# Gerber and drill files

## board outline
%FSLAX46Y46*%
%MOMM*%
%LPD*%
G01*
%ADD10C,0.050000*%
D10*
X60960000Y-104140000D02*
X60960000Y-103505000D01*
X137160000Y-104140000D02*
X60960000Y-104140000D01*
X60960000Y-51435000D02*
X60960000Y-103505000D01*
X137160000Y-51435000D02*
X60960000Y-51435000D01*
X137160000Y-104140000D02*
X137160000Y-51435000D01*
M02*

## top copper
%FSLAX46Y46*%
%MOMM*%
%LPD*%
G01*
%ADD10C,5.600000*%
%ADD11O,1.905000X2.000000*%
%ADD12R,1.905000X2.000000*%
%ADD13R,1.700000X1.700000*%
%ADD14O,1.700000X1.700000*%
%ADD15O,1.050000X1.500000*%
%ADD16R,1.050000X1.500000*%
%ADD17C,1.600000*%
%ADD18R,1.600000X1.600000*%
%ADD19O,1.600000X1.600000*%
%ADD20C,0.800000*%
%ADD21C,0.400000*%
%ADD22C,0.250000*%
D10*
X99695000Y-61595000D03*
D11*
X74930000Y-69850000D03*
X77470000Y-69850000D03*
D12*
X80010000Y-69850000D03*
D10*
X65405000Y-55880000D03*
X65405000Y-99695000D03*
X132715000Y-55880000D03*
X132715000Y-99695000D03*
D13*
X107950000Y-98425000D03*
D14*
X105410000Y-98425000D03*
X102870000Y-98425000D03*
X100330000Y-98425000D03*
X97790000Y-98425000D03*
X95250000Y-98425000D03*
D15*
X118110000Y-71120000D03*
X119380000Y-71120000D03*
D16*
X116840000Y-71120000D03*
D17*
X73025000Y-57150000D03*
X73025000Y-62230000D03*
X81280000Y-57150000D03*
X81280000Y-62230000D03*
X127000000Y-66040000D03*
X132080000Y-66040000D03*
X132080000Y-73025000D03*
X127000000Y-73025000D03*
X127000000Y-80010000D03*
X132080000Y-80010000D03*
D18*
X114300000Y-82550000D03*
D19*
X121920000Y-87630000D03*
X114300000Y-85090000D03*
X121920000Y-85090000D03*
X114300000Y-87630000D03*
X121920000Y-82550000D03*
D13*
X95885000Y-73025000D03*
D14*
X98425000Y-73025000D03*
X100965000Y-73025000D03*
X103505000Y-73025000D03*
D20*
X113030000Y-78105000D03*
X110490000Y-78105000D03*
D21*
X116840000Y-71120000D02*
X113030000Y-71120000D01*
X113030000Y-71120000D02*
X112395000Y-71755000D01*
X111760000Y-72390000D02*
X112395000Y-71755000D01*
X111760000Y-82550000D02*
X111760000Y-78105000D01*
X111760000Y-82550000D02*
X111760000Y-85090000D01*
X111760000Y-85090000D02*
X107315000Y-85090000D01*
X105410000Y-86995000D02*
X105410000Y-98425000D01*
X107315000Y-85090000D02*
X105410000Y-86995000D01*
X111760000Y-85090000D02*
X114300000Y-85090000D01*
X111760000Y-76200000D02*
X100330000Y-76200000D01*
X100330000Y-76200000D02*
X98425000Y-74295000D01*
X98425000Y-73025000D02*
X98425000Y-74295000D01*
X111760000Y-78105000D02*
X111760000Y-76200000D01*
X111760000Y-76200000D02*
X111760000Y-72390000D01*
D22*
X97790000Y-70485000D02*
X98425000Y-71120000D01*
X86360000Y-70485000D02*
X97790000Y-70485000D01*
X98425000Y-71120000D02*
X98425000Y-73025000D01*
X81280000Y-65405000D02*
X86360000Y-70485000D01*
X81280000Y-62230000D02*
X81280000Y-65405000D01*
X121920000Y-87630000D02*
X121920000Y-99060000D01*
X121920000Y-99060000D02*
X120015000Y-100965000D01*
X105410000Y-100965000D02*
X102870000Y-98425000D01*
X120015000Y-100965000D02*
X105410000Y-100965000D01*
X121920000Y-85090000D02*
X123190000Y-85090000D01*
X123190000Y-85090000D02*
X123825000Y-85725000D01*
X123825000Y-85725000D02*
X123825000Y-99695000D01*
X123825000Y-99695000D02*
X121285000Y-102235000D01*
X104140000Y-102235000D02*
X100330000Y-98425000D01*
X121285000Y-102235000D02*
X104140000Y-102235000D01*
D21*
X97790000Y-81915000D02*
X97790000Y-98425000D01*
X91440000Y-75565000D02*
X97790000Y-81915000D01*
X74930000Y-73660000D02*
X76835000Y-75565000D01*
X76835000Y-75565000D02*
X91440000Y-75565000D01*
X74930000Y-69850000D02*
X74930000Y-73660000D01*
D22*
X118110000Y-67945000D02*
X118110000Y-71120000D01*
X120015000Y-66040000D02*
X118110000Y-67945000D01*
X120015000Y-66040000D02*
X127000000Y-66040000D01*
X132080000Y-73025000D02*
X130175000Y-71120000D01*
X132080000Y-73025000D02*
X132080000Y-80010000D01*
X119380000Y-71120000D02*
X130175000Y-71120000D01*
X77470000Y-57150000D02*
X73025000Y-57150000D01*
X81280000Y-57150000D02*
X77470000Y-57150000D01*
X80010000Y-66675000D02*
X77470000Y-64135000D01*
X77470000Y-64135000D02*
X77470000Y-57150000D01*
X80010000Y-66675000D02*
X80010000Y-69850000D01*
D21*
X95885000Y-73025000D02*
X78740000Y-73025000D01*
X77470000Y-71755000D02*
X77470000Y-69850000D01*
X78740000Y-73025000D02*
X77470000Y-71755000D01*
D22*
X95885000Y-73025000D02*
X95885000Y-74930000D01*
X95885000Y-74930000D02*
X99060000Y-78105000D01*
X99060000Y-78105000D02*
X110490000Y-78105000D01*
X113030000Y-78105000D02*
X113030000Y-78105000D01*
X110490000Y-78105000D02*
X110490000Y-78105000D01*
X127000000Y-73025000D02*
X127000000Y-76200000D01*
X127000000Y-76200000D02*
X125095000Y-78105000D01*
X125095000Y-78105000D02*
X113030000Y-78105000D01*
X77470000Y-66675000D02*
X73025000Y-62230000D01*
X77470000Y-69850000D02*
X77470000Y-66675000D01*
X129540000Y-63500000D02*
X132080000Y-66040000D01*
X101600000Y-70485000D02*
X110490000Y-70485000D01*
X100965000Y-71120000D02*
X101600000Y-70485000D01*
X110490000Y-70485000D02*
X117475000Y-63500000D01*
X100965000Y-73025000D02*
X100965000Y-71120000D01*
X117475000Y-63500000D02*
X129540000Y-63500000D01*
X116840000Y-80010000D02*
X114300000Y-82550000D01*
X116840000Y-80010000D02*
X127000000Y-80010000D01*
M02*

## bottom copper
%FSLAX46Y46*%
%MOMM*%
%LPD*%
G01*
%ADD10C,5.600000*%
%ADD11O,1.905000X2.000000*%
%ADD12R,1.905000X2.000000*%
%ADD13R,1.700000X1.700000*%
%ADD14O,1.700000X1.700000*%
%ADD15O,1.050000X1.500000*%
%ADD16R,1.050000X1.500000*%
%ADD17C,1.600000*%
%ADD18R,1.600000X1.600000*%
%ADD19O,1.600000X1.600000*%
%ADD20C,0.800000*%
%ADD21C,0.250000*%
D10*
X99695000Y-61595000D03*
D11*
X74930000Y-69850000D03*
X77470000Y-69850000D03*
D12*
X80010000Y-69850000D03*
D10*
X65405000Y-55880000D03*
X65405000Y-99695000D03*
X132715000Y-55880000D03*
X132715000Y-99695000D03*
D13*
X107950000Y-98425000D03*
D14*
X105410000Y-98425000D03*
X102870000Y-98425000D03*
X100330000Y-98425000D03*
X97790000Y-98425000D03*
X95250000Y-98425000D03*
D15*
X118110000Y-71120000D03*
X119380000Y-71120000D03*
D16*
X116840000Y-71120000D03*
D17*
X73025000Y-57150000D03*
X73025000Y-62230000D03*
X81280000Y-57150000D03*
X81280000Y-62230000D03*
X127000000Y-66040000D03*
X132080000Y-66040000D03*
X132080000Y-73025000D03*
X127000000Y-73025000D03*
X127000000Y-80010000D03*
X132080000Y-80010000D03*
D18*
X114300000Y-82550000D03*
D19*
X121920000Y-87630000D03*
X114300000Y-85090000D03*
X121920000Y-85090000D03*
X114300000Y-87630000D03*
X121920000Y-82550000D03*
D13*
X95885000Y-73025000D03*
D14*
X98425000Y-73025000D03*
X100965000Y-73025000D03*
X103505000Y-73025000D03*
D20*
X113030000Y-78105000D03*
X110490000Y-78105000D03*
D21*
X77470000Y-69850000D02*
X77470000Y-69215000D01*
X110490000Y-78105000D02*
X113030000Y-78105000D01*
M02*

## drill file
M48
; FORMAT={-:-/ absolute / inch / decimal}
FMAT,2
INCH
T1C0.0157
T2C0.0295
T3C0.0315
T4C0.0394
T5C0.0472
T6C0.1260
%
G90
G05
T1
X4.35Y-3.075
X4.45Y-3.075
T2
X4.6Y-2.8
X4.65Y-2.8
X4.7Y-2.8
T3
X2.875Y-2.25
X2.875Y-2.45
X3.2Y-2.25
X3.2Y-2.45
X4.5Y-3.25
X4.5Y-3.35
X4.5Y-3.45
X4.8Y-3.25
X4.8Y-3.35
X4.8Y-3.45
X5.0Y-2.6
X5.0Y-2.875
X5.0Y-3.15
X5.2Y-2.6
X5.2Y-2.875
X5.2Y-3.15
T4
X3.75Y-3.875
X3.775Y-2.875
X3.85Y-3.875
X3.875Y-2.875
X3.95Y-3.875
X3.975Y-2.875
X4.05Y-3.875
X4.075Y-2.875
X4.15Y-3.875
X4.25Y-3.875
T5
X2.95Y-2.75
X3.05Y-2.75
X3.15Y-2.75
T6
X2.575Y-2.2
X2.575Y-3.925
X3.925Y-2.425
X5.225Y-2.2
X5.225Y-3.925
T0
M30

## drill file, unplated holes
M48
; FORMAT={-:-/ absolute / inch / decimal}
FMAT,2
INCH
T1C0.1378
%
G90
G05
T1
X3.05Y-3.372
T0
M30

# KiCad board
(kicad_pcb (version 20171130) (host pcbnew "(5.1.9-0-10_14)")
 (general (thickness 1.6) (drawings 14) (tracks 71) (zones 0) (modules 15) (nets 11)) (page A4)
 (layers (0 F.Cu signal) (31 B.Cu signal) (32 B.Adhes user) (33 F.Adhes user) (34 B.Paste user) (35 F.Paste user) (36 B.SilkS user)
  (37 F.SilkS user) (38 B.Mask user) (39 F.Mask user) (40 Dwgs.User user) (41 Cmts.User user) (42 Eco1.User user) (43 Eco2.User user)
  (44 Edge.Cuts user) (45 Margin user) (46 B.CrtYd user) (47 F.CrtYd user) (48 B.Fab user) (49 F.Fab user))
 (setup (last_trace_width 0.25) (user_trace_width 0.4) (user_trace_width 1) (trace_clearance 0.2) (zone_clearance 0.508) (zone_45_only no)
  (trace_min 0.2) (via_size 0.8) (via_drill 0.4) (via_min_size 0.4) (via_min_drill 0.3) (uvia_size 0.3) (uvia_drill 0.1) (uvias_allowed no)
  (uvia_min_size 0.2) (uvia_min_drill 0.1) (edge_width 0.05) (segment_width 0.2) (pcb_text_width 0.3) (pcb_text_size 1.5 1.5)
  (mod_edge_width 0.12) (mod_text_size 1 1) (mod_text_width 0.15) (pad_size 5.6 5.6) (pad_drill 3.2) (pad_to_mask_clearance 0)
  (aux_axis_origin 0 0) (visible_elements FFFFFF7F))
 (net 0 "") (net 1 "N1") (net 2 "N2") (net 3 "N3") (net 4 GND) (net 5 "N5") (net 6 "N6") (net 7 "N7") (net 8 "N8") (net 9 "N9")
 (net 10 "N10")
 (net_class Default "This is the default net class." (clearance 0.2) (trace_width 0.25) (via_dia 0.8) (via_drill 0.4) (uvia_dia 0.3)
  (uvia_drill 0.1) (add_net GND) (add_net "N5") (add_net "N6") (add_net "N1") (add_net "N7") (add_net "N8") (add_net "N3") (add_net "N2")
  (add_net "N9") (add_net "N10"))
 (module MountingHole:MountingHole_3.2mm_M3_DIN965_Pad (layer F.Cu) (at 99.695 61.595)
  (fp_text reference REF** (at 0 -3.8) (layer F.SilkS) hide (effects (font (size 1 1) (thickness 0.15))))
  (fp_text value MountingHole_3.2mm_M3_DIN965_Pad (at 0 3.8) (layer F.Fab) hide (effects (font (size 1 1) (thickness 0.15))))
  (pad "" thru_hole circle (at 0 0) (size 5.6 5.6) (drill 3.2) (layers *.Cu *.Mask)))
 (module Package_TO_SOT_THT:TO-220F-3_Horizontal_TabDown (layer F.Cu) (at 80.01 69.85 180)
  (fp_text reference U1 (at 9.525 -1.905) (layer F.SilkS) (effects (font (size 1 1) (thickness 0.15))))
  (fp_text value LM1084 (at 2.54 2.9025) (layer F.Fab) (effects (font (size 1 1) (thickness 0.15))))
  (pad 3 thru_hole oval (at 5.08 0 180) (size 1.905 2) (drill 1.2) (layers *.Cu *.Mask) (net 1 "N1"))
  (pad 2 thru_hole oval (at 2.54 0 180) (size 1.905 2) (drill 1.2) (layers *.Cu *.Mask) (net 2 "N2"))
  (pad 1 thru_hole rect (at 0 0 180) (size 1.905 2) (drill 1.2) (layers *.Cu *.Mask) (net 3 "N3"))
  (pad "" np_thru_hole oval (at 2.54 -15.8 180) (size 3.5 3.5) (drill 3.5) (layers *.Cu *.Mask)))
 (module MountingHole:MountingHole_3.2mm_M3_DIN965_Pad (layer F.Cu) (at 65.405 55.88)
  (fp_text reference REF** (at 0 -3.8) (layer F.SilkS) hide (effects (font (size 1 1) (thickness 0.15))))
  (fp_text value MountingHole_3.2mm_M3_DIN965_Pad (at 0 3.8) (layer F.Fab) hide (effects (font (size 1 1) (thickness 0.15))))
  (pad "" thru_hole circle (at 0 0) (size 5.6 5.6) (drill 3.2) (layers *.Cu *.Mask)))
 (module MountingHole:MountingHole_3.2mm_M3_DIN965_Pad (layer F.Cu) (at 65.405 99.695)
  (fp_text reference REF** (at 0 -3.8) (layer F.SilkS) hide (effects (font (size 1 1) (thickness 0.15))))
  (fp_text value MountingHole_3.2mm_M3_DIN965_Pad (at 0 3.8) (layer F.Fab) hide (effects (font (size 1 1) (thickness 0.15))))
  (pad "" thru_hole circle (at 0 0) (size 5.6 5.6) (drill 3.2) (layers *.Cu *.Mask)))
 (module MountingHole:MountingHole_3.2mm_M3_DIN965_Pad (layer F.Cu) (at 132.715 55.88)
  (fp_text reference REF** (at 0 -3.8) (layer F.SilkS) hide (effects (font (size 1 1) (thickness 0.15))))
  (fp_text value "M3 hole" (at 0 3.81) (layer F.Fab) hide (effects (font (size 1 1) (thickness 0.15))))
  (pad "" thru_hole circle (at 0 0) (size 5.6 5.6) (drill 3.2) (layers *.Cu *.Mask)))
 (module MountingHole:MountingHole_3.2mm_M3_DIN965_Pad (layer F.Cu) (at 132.715 99.695)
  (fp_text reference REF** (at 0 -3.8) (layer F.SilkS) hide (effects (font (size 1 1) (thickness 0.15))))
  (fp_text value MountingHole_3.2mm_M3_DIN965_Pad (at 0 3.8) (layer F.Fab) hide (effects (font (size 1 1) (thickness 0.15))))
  (pad "" thru_hole circle (at 0 0) (size 5.6 5.6) (drill 3.2) (layers *.Cu *.Mask)))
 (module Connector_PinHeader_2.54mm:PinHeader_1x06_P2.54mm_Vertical (layer F.Cu) (at 107.95 98.425 270)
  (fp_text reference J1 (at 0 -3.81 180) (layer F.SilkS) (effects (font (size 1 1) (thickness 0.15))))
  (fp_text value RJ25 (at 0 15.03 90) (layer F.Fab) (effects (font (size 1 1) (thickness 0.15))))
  (pad 1 thru_hole rect (at 0 0 270) (size 1.7 1.7) (drill 1) (layers *.Cu *.Mask))
  (pad 2 thru_hole oval (at 0 2.54 270) (size 1.7 1.7) (drill 1) (layers *.Cu *.Mask) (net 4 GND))
  (pad 3 thru_hole oval (at 0 5.08 270) (size 1.7 1.7) (drill 1) (layers *.Cu *.Mask) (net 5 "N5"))
  (pad 4 thru_hole oval (at 0 7.62 270) (size 1.7 1.7) (drill 1) (layers *.Cu *.Mask) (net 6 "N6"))
  (pad 5 thru_hole oval (at 0 10.16 270) (size 1.7 1.7) (drill 1) (layers *.Cu *.Mask) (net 1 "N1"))
  (pad 6 thru_hole oval (at 0 12.7 270) (size 1.7 1.7) (drill 1) (layers *.Cu *.Mask)))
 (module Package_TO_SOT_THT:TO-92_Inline (layer F.Cu) (at 116.84 71.12)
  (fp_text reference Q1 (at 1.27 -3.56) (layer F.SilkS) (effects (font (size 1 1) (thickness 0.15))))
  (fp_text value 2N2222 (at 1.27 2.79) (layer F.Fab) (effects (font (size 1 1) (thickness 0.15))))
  (pad 2 thru_hole oval (at 1.27 0) (size 1.05 1.5) (drill 0.75) (layers *.Cu *.Mask) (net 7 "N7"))
  (pad 3 thru_hole oval (at 2.54 0) (size 1.05 1.5) (drill 0.75) (layers *.Cu *.Mask) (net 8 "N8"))
  (pad 1 thru_hole rect (at 0 0) (size 1.05 1.5) (drill 0.75) (layers *.Cu *.Mask) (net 4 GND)))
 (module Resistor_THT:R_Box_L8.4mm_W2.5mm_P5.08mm (layer F.Cu) (at 73.025 57.15 270)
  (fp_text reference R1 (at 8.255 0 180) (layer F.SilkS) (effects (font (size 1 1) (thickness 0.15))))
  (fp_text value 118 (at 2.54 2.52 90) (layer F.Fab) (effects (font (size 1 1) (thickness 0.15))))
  (pad 1 thru_hole circle (at 0 0 270) (size 1.6 1.6) (drill 0.8) (layers *.Cu *.Mask) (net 3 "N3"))
  (pad 2 thru_hole circle (at 5.08 0 270) (size 1.6 1.6) (drill 0.8) (layers *.Cu *.Mask) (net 2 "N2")))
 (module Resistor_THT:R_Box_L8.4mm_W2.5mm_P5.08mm (layer F.Cu) (at 81.28 62.23 90)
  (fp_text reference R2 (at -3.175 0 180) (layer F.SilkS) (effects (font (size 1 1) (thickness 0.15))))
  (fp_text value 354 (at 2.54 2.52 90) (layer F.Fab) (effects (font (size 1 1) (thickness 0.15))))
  (pad 2 thru_hole circle (at 5.08 0 90) (size 1.6 1.6) (drill 0.8) (layers *.Cu *.Mask) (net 3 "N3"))
  (pad 1 thru_hole circle (at 0 0 90) (size 1.6 1.6) (drill 0.8) (layers *.Cu *.Mask) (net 4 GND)))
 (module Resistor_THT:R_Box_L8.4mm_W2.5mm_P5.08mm (layer F.Cu) (at 127 66.04)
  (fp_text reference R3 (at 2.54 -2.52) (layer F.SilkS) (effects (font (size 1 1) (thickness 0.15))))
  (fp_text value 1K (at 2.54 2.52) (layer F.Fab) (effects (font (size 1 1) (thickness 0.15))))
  (pad 1 thru_hole circle (at 0 0) (size 1.6 1.6) (drill 0.8) (layers *.Cu *.Mask) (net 7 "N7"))
  (pad 2 thru_hole circle (at 5.08 0) (size 1.6 1.6) (drill 0.8) (layers *.Cu *.Mask) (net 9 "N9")))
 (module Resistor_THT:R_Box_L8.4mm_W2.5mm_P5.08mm (layer F.Cu) (at 127 73.025)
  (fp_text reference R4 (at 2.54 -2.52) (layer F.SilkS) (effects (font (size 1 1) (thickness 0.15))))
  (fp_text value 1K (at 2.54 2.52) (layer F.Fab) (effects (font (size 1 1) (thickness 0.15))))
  (pad 2 thru_hole circle (at 5.08 0) (size 1.6 1.6) (drill 0.8) (layers *.Cu *.Mask) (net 8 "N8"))
  (pad 1 thru_hole circle (at 0 0) (size 1.6 1.6) (drill 0.8) (layers *.Cu *.Mask) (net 2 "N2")))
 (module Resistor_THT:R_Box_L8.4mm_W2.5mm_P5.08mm (layer F.Cu) (at 127 80.01)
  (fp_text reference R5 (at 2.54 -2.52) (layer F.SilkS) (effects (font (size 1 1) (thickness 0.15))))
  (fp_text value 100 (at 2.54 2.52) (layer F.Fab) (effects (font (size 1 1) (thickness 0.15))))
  (pad 1 thru_hole circle (at 0 0) (size 1.6 1.6) (drill 0.8) (layers *.Cu *.Mask) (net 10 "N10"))
  (pad 2 thru_hole circle (at 5.08 0) (size 1.6 1.6) (drill 0.8) (layers *.Cu *.Mask) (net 8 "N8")))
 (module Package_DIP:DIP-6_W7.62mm (layer F.Cu) (at 114.3 82.55)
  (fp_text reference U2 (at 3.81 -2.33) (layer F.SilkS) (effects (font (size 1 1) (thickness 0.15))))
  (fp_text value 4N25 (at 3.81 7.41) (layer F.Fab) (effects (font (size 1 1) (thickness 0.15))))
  (pad 1 thru_hole rect (at 0 0) (size 1.6 1.6) (drill 0.8) (layers *.Cu *.Mask) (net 10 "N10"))
  (pad 4 thru_hole oval (at 7.62 5.08) (size 1.6 1.6) (drill 0.8) (layers *.Cu *.Mask) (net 5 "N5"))
  (pad 2 thru_hole oval (at 0 2.54) (size 1.6 1.6) (drill 0.8) (layers *.Cu *.Mask) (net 4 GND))
  (pad 5 thru_hole oval (at 7.62 2.54) (size 1.6 1.6) (drill 0.8) (layers *.Cu *.Mask) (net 6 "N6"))
  (pad 3 thru_hole oval (at 0 5.08) (size 1.6 1.6) (drill 0.8) (layers *.Cu *.Mask))
  (pad 6 thru_hole oval (at 7.62 0) (size 1.6 1.6) (drill 0.8) (layers *.Cu *.Mask)))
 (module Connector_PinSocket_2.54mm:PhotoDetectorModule (layer F.Cu) (at 95.885 73.025 90)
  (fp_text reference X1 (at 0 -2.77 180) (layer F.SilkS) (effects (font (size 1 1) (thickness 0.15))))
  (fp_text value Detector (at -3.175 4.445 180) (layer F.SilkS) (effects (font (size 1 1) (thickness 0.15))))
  (pad 1 thru_hole rect (at 0 0 90) (size 1.7 1.7) (drill 1) (layers *.Cu *.Mask) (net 2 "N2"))
  (pad 2 thru_hole oval (at 0 2.54 90) (size 1.7 1.7) (drill 1) (layers *.Cu *.Mask) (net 4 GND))
  (pad 3 thru_hole oval (at 0 5.08 90) (size 1.7 1.7) (drill 1) (layers *.Cu *.Mask) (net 9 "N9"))
  (pad 4 thru_hole oval (at 0 7.62 90) (size 1.7 1.7) (drill 1) (layers *.Cu *.Mask)))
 (gr_line (start 60.96 104.14) (end 60.96 103.505) (layer Edge.Cuts) (width 0.05))
 (gr_line (start 137.16 104.14) (end 60.96 104.14) (layer Edge.Cuts) (width 0.05))
 (gr_line (start 60.96 51.435) (end 60.96 103.505) (layer Edge.Cuts) (width 0.05))
 (gr_line (start 137.16 51.435) (end 60.96 51.435) (layer Edge.Cuts) (width 0.05))
 (gr_line (start 137.16 104.14) (end 137.16 51.435) (layer Edge.Cuts) (width 0.05))
 (segment (start 116.84 71.12) (end 113.03 71.12) (width 0.4) (layer F.Cu) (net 4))
 (segment (start 113.03 71.12) (end 112.395 71.755) (width 0.4) (layer F.Cu) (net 4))
 (segment (start 111.76 72.39) (end 112.395 71.755) (width 0.4) (layer F.Cu) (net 4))
 (segment (start 111.76 82.55) (end 111.76 78.105) (width 0.4) (layer F.Cu) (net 4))
 (segment (start 111.76 82.55) (end 111.76 85.09) (width 0.4) (layer F.Cu) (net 4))
 (segment (start 111.76 85.09) (end 107.315 85.09) (width 0.4) (layer F.Cu) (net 4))
 (segment (start 105.41 86.995) (end 105.41 98.425) (width 0.4) (layer F.Cu) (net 4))
 (segment (start 107.315 85.09) (end 105.41 86.995) (width 0.4) (layer F.Cu) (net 4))
 (segment (start 111.76 85.09) (end 114.3 85.09) (width 0.4) (layer F.Cu) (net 4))
 (segment (start 111.76 76.2) (end 100.33 76.2) (width 0.4) (layer F.Cu) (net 4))
 (segment (start 100.33 76.2) (end 98.425 74.295) (width 0.4) (layer F.Cu) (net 4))
 (segment (start 98.425 73.025) (end 98.425 74.295) (width 0.4) (layer F.Cu) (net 4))
 (segment (start 111.76 78.105) (end 111.76 76.2) (width 0.4) (layer F.Cu) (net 4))
 (segment (start 111.76 76.2) (end 111.76 72.39) (width 0.4) (layer F.Cu) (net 4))
 (segment (start 97.79 70.485) (end 98.425 71.12) (width 0.25) (layer F.Cu) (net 4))
 (segment (start 86.36 70.485) (end 97.79 70.485) (width 0.25) (layer F.Cu) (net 4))
 (segment (start 98.425 71.12) (end 98.425 73.025) (width 0.25) (layer F.Cu) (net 4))
 (segment (start 81.28 65.405) (end 86.36 70.485) (width 0.25) (layer F.Cu) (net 4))
 (segment (start 81.28 62.23) (end 81.28 65.405) (width 0.25) (layer F.Cu) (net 4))
 (segment (start 121.92 87.63) (end 121.92 99.06) (width 0.25) (layer F.Cu) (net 5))
 (segment (start 121.92 99.06) (end 120.015 100.965) (width 0.25) (layer F.Cu) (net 5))
 (segment (start 105.41 100.965) (end 102.87 98.425) (width 0.25) (layer F.Cu) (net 5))
 (segment (start 120.015 100.965) (end 105.41 100.965) (width 0.25) (layer F.Cu) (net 5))
 (segment (start 121.92 85.09) (end 123.19 85.09) (width 0.25) (layer F.Cu) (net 6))
 (segment (start 123.19 85.09) (end 123.825 85.725) (width 0.25) (layer F.Cu) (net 6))
 (segment (start 123.825 85.725) (end 123.825 99.695) (width 0.25) (layer F.Cu) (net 6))
 (segment (start 123.825 99.695) (end 121.285 102.235) (width 0.25) (layer F.Cu) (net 6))
 (segment (start 104.14 102.235) (end 100.33 98.425) (width 0.25) (layer F.Cu) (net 6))
 (segment (start 121.285 102.235) (end 104.14 102.235) (width 0.25) (layer F.Cu) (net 6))
 (segment (start 97.79 81.915) (end 97.79 98.425) (width 0.4) (layer F.Cu) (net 1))
 (segment (start 91.44 75.565) (end 97.79 81.915) (width 0.4) (layer F.Cu) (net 1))
 (segment (start 74.93 73.66) (end 76.835 75.565) (width 0.4) (layer F.Cu) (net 1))
 (segment (start 76.835 75.565) (end 91.44 75.565) (width 0.4) (layer F.Cu) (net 1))
 (segment (start 74.93 69.85) (end 74.93 73.66) (width 0.4) (layer F.Cu) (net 1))
 (segment (start 118.11 67.945) (end 118.11 71.12) (width 0.25) (layer F.Cu) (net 7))
 (segment (start 120.015 66.04) (end 118.11 67.945) (width 0.25) (layer F.Cu) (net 7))
 (segment (start 120.015 66.04) (end 127 66.04) (width 0.25) (layer F.Cu) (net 7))
 (segment (start 132.08 73.025) (end 130.175 71.12) (width 0.25) (layer F.Cu) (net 8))
 (segment (start 132.08 73.025) (end 132.08 80.01) (width 0.25) (layer F.Cu) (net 8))
 (segment (start 119.38 71.12) (end 130.175 71.12) (width 0.25) (layer F.Cu) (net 8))
 (segment (start 77.47 57.15) (end 73.025 57.15) (width 0.25) (layer F.Cu) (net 3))
 (segment (start 81.28 57.15) (end 77.47 57.15) (width 0.25) (layer F.Cu) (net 3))
 (segment (start 80.01 69.85) (end 80.01 68.58) (width 0.25) (layer B.Cu) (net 3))
 (segment (start 80.01 66.675) (end 77.47 64.135) (width 0.25) (layer F.Cu) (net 3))
 (segment (start 77.47 64.135) (end 77.47 57.15) (width 0.25) (layer F.Cu) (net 3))
 (segment (start 80.01 68.58) (end 80.01 66.675) (width 0.25) (layer F.Cu) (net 3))
 (segment (start 95.885 73.025) (end 78.74 73.025) (width 0.4) (layer F.Cu) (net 2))
 (segment (start 77.47 71.755) (end 77.47 69.85) (width 0.4) (layer F.Cu) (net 2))
 (segment (start 78.74 73.025) (end 77.47 71.755) (width 0.4) (layer F.Cu) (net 2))
 (segment (start 77.47 69.85) (end 77.47 69.215) (width 0.25) (layer B.Cu) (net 2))
 (segment (start 95.885 73.025) (end 95.885 74.93) (width 0.25) (layer F.Cu) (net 2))
 (segment (start 95.885 74.93) (end 99.06 78.105) (width 0.25) (layer F.Cu) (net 2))
 (segment (start 99.06 78.105) (end 110.49 78.105) (width 0.25) (layer F.Cu) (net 2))
 (segment (start 113.03 78.105) (end 113.03 78.105) (width 0.25) (layer F.Cu) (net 2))
 (via (at 113.03 78.105) (size 0.8) (drill 0.4) (layers F.Cu B.Cu) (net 2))
 (segment (start 110.49 78.105) (end 110.49 78.105) (width 0.25) (layer F.Cu) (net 2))
 (via (at 110.49 78.105) (size 0.8) (drill 0.4) (layers F.Cu B.Cu) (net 2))
 (segment (start 110.49 78.105) (end 113.03 78.105) (width 0.25) (layer B.Cu) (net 2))
 (segment (start 127 73.025) (end 127 76.2) (width 0.25) (layer F.Cu) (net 2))
 (segment (start 127 76.2) (end 125.095 78.105) (width 0.25) (layer F.Cu) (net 2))
 (segment (start 125.095 78.105) (end 113.03 78.105) (width 0.25) (layer F.Cu) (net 2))
 (segment (start 77.47 66.675) (end 73.025 62.23) (width 0.25) (layer F.Cu) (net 2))
 (segment (start 77.47 69.85) (end 77.47 66.675) (width 0.25) (layer F.Cu) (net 2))
 (segment (start 129.54 63.5) (end 132.08 66.04) (width 0.25) (layer F.Cu) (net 9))
 (segment (start 101.6 70.485) (end 110.49 70.485) (width 0.25) (layer F.Cu) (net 9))
 (segment (start 100.965 71.12) (end 101.6 70.485) (width 0.25) (layer F.Cu) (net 9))
 (segment (start 110.49 70.485) (end 117.475 63.5) (width 0.25) (layer F.Cu) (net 9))
 (segment (start 100.965 73.025) (end 100.965 71.12) (width 0.25) (layer F.Cu) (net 9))
 (segment (start 117.475 63.5) (end 129.54 63.5) (width 0.25) (layer F.Cu) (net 9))
 (segment (start 116.84 80.01) (end 114.3 82.55) (width 0.25) (layer F.Cu) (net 10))
 (segment (start 116.84 80.01) (end 127 80.01) (width 0.25) (layer F.Cu) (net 10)))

